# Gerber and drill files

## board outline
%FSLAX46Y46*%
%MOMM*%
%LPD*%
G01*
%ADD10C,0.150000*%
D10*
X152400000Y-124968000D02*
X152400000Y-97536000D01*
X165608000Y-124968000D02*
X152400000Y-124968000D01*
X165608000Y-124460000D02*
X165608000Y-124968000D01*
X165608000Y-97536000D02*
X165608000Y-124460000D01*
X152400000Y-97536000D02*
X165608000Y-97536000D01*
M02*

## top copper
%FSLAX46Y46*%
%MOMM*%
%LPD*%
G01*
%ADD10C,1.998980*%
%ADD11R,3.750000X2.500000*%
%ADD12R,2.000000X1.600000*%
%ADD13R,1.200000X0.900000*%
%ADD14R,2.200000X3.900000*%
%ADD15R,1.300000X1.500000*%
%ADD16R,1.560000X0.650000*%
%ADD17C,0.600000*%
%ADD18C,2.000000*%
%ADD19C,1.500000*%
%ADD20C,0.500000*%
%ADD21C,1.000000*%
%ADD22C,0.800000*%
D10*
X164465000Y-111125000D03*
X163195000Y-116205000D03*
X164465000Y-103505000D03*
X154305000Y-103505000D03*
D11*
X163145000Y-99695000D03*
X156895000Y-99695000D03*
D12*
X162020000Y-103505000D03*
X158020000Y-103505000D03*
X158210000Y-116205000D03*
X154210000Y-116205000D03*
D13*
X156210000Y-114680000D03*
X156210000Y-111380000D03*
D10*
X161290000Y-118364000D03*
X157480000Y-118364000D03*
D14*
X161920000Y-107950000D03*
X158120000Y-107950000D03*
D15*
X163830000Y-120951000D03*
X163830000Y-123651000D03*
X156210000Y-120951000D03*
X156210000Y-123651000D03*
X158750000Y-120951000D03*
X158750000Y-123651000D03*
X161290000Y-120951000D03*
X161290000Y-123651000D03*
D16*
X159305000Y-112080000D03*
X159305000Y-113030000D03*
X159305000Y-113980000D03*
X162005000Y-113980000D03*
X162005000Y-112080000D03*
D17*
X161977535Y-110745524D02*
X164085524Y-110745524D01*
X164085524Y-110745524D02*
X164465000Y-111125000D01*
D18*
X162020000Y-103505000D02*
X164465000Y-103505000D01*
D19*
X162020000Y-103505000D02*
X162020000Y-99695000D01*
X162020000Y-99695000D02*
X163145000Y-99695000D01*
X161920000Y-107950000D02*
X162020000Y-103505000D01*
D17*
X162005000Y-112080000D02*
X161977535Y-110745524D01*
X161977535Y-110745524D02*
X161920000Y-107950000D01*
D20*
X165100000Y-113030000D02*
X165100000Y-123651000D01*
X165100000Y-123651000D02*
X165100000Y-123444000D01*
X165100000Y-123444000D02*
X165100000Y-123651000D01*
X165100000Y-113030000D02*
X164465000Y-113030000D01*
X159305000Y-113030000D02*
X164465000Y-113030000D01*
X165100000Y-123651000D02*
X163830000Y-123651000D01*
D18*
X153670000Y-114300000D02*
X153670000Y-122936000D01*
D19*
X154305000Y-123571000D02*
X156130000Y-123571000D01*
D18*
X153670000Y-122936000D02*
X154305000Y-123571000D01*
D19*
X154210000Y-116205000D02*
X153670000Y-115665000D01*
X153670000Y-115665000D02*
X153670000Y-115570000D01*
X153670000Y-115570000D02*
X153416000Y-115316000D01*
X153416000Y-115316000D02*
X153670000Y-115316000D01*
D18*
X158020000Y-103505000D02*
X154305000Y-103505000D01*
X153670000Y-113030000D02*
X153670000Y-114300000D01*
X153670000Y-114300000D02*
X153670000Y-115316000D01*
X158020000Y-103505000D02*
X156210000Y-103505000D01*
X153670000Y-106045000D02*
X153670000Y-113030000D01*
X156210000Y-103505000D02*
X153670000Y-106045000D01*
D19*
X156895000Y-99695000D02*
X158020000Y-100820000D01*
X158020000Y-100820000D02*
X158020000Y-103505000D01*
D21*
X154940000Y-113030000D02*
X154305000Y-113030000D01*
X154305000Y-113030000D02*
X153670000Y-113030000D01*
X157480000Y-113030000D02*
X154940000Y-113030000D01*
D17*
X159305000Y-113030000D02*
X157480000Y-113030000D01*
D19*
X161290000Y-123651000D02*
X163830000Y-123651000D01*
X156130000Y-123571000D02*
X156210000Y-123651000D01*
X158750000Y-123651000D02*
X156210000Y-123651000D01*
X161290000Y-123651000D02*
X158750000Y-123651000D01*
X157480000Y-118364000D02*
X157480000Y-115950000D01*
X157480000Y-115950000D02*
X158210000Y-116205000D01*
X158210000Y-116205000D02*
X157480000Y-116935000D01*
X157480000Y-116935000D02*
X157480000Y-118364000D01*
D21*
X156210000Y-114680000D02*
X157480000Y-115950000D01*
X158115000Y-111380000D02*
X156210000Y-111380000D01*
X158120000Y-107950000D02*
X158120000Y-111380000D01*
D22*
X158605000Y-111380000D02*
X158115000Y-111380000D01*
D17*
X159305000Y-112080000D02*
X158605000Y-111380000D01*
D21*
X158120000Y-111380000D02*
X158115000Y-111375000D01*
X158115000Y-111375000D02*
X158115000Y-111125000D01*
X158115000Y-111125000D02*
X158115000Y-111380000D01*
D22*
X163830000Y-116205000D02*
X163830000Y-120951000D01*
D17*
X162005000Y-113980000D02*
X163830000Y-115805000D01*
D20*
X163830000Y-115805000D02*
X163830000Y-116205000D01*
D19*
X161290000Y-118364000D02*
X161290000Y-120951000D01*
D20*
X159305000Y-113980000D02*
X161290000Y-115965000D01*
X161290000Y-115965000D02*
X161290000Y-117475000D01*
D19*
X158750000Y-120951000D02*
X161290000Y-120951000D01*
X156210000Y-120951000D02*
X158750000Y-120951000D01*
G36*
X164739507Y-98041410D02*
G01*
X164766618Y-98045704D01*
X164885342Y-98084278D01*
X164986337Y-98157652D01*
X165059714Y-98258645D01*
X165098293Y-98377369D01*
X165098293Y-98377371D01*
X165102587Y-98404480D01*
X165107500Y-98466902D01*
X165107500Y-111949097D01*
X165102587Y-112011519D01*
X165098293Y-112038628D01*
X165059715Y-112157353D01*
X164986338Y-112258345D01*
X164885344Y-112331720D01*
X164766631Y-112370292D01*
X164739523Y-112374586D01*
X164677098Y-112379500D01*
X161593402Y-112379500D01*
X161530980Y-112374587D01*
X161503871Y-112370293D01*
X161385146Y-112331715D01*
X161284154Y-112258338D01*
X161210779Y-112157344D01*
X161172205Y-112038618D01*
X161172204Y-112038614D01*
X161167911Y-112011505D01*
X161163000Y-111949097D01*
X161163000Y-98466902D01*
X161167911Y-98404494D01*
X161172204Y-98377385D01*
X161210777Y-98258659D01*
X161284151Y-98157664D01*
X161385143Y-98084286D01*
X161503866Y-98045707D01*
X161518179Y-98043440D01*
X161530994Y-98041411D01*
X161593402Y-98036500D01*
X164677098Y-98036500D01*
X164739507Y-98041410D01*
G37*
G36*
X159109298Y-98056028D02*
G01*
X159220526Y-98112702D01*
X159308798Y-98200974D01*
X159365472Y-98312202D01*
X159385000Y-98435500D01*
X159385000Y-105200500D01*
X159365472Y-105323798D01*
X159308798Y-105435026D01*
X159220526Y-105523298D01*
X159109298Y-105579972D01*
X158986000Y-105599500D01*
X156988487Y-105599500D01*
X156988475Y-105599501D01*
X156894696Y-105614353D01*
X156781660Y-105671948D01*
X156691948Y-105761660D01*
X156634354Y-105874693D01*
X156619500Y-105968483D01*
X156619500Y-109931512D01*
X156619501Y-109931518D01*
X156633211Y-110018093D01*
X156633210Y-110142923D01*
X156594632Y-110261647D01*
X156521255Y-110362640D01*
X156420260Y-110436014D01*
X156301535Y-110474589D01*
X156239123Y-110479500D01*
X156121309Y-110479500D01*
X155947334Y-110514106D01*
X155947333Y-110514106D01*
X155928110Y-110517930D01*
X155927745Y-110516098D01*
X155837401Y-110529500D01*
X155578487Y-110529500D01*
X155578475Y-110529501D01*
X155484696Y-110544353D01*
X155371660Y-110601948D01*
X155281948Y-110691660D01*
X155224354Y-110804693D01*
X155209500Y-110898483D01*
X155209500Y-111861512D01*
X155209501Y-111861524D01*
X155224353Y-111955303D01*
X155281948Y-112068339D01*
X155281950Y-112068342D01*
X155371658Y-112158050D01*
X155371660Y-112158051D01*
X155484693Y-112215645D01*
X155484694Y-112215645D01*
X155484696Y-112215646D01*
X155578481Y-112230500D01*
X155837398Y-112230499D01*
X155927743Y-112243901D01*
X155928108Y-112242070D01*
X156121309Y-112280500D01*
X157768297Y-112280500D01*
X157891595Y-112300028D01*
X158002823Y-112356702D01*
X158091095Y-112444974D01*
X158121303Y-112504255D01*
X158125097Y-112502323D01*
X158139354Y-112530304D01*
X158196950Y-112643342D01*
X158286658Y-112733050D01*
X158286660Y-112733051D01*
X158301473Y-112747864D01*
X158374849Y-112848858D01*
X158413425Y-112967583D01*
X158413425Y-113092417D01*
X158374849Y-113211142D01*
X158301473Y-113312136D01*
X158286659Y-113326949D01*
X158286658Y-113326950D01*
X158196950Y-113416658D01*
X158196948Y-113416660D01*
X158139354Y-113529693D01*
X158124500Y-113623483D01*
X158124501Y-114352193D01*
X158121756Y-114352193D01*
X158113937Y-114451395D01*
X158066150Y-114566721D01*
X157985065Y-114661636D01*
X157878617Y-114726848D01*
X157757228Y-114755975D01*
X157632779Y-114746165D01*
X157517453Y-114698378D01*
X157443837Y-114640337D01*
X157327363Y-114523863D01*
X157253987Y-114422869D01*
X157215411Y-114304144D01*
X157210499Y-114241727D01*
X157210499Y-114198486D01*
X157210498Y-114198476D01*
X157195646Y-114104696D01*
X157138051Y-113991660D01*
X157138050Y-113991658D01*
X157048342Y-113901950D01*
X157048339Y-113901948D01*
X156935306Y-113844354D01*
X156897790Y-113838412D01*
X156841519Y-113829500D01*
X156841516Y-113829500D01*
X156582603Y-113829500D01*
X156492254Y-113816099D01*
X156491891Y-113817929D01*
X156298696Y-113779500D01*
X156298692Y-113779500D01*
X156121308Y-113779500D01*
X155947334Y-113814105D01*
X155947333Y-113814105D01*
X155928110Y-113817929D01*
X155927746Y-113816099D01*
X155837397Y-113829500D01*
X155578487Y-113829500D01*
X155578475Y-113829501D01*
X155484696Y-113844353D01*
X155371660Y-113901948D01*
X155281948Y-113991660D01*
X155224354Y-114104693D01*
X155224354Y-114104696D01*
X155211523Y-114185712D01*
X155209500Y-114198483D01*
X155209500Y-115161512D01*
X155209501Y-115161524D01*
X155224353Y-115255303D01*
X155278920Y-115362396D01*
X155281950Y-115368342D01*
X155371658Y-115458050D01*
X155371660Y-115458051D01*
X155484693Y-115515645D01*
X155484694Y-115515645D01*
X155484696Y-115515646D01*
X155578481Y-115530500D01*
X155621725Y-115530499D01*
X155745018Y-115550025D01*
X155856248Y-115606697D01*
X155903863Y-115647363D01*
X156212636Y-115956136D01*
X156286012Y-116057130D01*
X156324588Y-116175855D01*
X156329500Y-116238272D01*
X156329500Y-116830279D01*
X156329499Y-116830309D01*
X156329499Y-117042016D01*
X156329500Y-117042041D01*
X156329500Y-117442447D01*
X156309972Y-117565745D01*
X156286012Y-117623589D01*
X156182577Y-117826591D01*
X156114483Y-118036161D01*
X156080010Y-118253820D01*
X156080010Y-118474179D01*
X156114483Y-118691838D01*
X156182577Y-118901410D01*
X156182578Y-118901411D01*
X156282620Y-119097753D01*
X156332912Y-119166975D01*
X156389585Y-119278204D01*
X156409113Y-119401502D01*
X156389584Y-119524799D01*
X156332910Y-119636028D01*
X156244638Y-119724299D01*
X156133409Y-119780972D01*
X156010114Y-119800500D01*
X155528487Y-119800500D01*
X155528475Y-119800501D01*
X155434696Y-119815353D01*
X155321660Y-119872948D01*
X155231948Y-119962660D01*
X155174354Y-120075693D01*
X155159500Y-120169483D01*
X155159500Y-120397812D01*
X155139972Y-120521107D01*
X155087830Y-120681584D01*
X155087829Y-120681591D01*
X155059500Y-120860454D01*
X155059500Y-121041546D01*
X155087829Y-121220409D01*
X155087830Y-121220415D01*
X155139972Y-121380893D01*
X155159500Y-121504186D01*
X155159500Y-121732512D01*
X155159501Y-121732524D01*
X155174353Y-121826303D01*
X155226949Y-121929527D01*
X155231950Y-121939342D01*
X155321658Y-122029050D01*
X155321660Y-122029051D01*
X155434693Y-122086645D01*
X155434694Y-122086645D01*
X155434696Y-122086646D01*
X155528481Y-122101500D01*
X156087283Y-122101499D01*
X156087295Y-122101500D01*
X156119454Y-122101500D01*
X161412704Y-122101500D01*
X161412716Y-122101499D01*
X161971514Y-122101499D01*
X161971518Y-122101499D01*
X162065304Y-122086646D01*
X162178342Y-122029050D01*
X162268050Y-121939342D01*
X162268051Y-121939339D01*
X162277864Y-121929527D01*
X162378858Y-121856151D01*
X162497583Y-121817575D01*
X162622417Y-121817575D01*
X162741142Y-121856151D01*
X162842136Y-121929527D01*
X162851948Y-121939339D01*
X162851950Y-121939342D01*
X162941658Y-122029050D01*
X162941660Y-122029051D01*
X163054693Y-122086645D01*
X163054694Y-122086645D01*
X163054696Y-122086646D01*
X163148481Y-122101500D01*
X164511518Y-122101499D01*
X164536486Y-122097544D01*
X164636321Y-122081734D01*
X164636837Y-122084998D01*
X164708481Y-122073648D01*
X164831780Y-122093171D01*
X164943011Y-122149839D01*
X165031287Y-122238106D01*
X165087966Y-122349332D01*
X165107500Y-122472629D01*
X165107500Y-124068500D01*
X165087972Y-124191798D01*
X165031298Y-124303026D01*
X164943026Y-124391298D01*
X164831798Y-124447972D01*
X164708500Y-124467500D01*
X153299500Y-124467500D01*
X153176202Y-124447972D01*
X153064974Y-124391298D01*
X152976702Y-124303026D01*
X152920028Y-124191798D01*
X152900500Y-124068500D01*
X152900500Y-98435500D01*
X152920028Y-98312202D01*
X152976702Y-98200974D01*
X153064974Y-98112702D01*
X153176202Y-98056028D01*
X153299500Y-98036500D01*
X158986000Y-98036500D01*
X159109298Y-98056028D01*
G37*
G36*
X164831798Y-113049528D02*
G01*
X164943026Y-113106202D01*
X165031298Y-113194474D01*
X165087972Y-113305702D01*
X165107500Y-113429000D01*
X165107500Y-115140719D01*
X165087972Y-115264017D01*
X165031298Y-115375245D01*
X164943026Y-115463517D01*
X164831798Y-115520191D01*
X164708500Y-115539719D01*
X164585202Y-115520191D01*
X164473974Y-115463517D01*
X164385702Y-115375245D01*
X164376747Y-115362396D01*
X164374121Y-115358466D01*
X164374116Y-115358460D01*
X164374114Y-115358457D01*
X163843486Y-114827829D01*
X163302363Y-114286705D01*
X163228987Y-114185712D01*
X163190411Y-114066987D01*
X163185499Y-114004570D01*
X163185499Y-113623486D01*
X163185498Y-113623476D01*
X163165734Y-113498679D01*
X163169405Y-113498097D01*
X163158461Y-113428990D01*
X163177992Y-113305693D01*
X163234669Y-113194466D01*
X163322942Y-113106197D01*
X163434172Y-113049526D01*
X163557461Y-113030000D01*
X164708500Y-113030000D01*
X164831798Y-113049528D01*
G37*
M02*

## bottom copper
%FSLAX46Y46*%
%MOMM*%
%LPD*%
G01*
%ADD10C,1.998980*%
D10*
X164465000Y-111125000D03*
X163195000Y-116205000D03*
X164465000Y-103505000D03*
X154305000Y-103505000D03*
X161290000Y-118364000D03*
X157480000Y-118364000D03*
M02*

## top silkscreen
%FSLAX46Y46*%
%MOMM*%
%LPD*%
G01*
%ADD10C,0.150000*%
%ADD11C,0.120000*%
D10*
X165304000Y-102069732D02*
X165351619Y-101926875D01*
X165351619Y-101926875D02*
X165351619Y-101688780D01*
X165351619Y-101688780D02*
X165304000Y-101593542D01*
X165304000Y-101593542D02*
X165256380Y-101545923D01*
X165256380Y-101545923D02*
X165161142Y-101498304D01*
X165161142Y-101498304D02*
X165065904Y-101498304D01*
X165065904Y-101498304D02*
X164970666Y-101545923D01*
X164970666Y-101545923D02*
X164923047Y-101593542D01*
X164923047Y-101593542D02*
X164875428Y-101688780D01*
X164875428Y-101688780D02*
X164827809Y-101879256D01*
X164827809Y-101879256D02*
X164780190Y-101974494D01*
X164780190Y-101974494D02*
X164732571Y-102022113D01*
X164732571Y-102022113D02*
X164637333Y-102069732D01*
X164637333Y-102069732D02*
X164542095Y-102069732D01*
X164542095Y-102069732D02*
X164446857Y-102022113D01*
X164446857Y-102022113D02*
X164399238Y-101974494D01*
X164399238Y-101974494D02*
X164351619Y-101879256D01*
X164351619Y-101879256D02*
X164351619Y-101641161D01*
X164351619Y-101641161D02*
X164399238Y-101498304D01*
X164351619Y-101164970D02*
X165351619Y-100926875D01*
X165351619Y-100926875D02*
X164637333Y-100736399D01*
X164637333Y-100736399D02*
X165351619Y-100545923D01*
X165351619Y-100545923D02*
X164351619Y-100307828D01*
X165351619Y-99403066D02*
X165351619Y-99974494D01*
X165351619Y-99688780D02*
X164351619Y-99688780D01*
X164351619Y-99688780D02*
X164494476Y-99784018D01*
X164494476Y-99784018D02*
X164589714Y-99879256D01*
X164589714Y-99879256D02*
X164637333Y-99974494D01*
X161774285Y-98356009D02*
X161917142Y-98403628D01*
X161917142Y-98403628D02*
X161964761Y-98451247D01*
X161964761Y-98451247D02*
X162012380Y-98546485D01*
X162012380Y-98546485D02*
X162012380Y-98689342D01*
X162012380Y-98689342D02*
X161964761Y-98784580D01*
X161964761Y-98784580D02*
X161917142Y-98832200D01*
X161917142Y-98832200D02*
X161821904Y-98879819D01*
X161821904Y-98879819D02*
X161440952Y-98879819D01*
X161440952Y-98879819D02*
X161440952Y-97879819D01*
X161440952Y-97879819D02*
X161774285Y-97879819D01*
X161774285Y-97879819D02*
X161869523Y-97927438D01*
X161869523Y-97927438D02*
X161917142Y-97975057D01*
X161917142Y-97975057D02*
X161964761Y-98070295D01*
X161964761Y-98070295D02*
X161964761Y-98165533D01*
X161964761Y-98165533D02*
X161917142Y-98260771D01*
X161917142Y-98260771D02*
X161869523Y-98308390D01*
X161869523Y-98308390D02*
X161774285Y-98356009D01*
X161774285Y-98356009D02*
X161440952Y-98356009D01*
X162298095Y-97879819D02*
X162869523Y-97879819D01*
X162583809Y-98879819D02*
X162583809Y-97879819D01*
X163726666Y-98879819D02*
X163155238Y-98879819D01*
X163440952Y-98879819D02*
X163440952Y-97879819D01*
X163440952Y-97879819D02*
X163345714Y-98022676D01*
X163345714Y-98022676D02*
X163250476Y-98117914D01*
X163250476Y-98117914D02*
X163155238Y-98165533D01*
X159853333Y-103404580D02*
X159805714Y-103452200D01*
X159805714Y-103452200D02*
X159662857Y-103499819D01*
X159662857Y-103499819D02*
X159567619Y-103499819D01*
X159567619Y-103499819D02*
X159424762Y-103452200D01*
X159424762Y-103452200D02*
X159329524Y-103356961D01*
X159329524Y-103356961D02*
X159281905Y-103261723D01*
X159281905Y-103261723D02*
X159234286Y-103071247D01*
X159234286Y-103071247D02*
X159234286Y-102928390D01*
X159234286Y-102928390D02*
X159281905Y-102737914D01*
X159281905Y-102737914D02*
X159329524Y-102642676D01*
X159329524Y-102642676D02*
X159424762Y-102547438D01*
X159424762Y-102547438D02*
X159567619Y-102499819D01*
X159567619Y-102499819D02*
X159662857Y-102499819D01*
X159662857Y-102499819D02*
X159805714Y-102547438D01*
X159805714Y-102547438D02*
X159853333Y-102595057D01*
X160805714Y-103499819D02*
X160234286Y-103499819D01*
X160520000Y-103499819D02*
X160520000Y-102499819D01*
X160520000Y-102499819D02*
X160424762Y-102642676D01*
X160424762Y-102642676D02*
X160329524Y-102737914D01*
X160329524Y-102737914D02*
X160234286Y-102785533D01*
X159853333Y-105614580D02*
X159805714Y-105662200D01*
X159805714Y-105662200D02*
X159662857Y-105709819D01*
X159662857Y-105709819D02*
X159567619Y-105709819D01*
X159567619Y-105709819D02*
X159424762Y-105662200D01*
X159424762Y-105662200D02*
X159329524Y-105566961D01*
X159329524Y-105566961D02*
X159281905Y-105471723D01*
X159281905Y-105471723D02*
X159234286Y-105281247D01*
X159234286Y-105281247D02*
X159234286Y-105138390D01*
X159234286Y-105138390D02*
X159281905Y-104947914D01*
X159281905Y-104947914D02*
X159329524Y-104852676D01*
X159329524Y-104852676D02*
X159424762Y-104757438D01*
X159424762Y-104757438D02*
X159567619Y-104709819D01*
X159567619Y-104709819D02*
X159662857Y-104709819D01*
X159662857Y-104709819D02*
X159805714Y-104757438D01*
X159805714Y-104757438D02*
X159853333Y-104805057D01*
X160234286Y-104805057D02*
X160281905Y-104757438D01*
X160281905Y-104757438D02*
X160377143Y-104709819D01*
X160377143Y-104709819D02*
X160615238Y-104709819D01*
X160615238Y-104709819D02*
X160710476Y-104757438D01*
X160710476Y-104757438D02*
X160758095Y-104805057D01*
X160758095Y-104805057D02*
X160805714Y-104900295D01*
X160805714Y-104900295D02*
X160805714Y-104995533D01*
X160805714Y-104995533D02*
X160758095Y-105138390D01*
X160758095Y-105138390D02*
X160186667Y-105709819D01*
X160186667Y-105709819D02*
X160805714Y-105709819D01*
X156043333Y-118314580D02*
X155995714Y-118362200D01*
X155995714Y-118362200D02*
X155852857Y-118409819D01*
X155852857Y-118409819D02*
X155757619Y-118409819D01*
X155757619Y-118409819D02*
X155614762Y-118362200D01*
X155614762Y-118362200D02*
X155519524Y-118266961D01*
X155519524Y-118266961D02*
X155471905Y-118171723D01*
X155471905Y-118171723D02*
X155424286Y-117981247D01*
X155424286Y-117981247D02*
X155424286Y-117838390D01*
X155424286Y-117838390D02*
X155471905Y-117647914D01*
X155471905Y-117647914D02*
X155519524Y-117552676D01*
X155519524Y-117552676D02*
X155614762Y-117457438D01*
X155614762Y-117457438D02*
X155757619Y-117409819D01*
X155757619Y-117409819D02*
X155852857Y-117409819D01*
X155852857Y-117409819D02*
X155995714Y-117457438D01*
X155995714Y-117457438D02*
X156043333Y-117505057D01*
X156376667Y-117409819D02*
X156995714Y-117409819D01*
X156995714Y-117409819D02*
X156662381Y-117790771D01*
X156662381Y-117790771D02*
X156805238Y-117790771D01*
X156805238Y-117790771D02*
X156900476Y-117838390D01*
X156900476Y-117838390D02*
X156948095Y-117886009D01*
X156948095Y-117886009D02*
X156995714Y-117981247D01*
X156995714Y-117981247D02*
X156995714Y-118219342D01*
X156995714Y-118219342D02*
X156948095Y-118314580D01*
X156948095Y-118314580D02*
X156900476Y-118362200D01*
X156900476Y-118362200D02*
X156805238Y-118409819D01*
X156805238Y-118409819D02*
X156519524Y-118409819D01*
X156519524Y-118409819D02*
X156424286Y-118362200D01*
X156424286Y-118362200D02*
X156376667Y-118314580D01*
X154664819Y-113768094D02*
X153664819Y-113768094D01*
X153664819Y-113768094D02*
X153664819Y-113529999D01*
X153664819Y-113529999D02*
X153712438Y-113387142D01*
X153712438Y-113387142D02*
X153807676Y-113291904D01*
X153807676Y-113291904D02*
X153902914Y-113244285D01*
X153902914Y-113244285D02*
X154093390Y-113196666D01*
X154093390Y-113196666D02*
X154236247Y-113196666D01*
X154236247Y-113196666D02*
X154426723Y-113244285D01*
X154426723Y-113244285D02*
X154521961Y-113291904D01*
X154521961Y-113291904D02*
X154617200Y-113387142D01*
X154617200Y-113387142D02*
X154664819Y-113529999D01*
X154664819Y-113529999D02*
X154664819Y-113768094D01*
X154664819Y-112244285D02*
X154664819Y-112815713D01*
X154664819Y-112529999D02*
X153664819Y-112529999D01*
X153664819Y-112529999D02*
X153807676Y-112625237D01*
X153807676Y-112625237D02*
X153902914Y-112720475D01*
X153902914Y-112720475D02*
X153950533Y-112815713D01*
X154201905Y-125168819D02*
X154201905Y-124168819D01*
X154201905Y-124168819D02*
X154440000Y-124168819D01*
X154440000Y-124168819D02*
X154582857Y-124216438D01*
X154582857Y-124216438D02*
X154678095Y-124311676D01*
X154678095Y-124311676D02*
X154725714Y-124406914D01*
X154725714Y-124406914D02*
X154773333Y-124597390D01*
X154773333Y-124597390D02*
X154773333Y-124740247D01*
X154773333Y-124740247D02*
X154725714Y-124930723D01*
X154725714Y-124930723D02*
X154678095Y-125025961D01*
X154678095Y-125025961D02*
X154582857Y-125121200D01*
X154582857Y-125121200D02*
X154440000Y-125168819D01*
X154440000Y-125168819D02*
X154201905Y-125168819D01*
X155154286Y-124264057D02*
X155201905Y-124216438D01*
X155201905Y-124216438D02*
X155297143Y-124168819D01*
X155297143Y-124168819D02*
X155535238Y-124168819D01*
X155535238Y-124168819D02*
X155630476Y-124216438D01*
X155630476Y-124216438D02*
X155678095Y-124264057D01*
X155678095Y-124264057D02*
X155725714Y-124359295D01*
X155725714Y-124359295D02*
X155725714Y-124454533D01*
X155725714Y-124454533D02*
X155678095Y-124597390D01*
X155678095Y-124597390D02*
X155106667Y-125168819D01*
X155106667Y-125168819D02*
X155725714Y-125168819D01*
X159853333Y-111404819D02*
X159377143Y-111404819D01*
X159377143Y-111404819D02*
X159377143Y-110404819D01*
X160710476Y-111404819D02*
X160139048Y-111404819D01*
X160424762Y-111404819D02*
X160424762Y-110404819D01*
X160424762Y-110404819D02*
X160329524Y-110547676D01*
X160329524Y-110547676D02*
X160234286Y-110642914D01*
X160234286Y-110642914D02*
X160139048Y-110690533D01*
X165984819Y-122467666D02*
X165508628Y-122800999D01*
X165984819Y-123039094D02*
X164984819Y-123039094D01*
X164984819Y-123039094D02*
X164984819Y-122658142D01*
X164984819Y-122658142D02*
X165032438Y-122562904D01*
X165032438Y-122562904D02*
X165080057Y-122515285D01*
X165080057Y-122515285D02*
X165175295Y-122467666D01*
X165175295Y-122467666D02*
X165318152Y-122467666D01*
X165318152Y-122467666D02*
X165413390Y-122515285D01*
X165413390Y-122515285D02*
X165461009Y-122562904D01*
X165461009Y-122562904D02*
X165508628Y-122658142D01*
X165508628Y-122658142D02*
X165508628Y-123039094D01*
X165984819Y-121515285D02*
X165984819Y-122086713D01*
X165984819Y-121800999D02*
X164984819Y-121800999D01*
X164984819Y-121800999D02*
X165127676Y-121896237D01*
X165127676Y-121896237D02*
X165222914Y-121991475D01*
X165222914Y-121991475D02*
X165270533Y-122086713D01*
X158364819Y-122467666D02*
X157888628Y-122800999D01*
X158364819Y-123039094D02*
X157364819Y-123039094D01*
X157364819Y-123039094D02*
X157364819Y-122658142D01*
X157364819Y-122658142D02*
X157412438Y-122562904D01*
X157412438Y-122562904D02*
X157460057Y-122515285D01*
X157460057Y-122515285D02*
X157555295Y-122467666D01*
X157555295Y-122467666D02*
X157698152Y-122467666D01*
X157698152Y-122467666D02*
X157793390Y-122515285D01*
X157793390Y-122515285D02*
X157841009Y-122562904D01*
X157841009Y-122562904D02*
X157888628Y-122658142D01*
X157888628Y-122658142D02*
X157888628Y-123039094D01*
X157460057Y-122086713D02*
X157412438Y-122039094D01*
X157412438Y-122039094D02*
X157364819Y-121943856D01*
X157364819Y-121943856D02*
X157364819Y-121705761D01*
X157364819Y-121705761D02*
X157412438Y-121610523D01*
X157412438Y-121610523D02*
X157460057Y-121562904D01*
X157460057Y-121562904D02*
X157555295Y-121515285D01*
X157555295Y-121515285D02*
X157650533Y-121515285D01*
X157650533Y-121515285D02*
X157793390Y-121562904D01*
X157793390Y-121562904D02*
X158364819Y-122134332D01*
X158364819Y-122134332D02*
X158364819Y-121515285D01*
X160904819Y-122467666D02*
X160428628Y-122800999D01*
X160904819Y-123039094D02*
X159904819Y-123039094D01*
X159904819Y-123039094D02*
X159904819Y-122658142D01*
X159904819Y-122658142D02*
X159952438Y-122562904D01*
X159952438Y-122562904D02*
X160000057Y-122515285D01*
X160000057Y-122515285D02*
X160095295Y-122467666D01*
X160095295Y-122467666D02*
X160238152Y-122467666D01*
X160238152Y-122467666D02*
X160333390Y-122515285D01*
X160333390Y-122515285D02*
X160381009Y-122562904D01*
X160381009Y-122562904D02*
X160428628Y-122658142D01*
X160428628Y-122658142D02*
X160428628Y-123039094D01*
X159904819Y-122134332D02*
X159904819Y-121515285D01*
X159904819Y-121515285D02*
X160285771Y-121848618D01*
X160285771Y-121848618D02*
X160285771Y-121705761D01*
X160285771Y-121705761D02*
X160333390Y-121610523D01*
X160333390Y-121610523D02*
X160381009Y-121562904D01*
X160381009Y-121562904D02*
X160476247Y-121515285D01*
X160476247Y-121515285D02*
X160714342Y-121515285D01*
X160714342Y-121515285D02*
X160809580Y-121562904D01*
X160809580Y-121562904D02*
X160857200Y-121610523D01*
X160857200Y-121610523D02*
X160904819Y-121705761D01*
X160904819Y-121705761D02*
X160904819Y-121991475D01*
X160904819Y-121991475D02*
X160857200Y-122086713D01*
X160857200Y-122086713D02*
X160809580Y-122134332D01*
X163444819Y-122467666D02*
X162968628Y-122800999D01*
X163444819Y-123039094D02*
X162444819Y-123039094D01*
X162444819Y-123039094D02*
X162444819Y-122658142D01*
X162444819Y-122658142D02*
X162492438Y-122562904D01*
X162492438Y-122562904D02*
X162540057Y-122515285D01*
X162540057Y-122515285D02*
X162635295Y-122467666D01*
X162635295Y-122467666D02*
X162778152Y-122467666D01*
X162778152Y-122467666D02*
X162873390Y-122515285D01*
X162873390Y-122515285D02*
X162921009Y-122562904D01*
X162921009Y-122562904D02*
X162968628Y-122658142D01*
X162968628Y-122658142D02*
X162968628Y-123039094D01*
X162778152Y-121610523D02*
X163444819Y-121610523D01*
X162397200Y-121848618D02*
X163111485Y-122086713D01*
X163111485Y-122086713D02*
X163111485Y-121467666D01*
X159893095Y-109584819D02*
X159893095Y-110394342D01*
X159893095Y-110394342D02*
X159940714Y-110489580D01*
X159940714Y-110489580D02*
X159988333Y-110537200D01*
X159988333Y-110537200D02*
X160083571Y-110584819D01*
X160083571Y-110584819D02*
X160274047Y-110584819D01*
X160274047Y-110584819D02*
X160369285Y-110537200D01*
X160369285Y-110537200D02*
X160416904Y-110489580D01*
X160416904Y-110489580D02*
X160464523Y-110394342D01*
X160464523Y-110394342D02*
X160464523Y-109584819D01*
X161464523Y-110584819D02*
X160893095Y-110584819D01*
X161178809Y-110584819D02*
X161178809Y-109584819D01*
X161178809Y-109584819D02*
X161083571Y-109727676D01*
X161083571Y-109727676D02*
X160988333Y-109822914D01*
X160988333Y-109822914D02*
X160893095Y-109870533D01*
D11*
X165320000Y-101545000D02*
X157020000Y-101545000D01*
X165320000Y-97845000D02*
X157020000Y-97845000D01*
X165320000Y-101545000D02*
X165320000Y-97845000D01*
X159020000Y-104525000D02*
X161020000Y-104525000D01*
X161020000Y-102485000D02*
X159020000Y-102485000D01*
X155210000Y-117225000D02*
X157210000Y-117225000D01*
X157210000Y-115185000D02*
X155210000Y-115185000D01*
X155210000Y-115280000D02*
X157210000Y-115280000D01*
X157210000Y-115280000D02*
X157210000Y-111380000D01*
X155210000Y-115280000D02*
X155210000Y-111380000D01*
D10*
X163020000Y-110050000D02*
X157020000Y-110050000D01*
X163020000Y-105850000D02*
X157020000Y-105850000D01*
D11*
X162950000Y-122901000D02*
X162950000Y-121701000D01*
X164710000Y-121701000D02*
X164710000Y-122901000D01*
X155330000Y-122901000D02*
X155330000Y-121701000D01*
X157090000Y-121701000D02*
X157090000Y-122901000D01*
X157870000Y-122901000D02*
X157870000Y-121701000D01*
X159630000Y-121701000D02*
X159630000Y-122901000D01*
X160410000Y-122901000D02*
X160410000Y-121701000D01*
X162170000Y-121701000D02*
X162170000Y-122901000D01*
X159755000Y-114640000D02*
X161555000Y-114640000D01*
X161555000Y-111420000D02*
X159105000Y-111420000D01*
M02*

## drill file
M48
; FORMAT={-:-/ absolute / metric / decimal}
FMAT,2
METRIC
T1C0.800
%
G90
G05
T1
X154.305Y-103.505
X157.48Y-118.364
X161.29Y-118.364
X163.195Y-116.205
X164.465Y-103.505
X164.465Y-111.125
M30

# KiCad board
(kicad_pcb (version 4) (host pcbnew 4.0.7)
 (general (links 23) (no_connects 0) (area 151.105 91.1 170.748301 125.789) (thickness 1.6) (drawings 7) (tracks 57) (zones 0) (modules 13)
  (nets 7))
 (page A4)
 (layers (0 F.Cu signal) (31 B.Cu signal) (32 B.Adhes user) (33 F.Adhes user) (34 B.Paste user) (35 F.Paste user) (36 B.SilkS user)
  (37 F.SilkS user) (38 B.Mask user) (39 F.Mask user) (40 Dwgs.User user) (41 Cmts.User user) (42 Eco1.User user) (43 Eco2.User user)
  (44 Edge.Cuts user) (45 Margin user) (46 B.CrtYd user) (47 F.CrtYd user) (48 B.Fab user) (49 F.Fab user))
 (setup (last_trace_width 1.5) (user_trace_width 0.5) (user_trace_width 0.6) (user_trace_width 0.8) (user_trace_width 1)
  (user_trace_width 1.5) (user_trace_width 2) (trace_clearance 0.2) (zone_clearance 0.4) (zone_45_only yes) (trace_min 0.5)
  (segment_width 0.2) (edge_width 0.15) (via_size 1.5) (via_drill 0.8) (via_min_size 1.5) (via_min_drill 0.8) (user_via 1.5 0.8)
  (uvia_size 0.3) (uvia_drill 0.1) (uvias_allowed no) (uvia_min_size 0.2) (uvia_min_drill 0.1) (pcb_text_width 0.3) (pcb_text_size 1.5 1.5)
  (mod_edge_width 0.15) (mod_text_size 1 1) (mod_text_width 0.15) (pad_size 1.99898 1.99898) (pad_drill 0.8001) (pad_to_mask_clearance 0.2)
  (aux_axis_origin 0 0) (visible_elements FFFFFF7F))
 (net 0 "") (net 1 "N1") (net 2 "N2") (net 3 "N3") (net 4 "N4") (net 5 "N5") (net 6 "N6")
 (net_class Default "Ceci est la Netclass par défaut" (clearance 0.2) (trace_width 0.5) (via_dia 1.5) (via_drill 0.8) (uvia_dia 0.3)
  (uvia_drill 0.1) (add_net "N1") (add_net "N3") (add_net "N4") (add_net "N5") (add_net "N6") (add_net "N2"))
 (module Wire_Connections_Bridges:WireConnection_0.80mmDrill (layer F.Cu) (at 165.1 95.885 270)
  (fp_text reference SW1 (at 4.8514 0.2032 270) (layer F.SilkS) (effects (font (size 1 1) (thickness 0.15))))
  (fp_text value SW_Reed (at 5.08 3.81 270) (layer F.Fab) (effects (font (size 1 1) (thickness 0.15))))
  (pad 1 thru_hole circle (at 15.24 0.635 270) (size 1.99898 1.99898) (drill 0.8001) (layers *.Cu *.Mask) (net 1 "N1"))
  (pad 2 thru_hole circle (at 20.32 1.905 270) (size 1.99898 1.99898) (drill 0.8001) (layers *.Cu *.Mask) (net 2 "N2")))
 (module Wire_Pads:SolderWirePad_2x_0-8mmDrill (layer F.Cu) (at 162.56 94.615 180)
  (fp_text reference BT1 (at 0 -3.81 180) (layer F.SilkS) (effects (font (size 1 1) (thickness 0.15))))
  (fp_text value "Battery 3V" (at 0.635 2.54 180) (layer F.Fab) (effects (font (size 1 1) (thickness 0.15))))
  (pad 1 thru_hole circle (at -1.905 -8.89 180) (size 1.99898 1.99898) (drill 0.8001) (layers *.Cu *.Mask) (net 1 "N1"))
  (pad 2 thru_hole circle (at 8.255 -8.89 180) (size 1.99898 1.99898) (drill 0.8001) (layers *.Cu *.Mask) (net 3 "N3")))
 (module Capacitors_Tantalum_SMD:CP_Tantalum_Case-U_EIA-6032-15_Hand (layer F.Cu) (at 160.02 99.695 180)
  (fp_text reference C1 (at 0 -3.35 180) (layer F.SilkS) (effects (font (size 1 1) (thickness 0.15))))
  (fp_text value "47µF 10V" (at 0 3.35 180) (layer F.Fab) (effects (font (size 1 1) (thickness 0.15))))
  (fp_line (start -5.3 -1.85) (end 3 -1.85) (layer F.SilkS) (width 0.12))
  (fp_line (start -5.3 1.85) (end 3 1.85) (layer F.SilkS) (width 0.12))
  (fp_line (start -5.3 -1.85) (end -5.3 1.85) (layer F.SilkS) (width 0.12))
  (pad 1 smd rect (at -3.125 0 180) (size 3.75 2.5) (layers F.Cu F.Paste F.Mask) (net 1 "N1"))
  (pad 2 smd rect (at 3.125 0 180) (size 3.75 2.5) (layers F.Cu F.Paste F.Mask) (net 3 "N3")))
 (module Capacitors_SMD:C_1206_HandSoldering (layer F.Cu) (at 160.02 103.505 180)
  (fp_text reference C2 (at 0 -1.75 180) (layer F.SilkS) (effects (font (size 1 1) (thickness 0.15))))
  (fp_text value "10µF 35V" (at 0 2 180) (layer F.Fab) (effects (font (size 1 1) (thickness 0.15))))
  (fp_line (start 1 -1.02) (end -1 -1.02) (layer F.SilkS) (width 0.12))
  (fp_line (start -1 1.02) (end 1 1.02) (layer F.SilkS) (width 0.12))
  (pad 1 smd rect (at -2 0 180) (size 2 1.6) (layers F.Cu F.Paste F.Mask) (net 1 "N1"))
  (pad 2 smd rect (at 2 0 180) (size 2 1.6) (layers F.Cu F.Paste F.Mask) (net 3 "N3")))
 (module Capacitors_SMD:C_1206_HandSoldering (layer F.Cu) (at 156.21 116.205 180)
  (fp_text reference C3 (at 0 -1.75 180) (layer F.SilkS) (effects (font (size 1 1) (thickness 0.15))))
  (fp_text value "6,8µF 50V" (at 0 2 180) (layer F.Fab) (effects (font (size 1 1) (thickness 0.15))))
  (fp_line (start 1 -1.02) (end -1 -1.02) (layer F.SilkS) (width 0.12))
  (fp_line (start -1 1.02) (end 1 1.02) (layer F.SilkS) (width 0.12))
  (pad 1 smd rect (at -2 0 180) (size 2 1.6) (layers F.Cu F.Paste F.Mask) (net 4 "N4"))
  (pad 2 smd rect (at 2 0 180) (size 2 1.6) (layers F.Cu F.Paste F.Mask) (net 3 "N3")))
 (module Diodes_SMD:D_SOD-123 (layer F.Cu) (at 156.21 113.03 90)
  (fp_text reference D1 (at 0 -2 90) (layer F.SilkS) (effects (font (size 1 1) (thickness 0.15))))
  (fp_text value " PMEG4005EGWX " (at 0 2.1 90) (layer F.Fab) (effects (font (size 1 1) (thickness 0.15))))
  (fp_line (start -2.25 -1) (end -2.25 1) (layer F.SilkS) (width 0.12))
  (fp_line (start -2.25 1) (end 1.65 1) (layer F.SilkS) (width 0.12))
  (fp_line (start -2.25 -1) (end 1.65 -1) (layer F.SilkS) (width 0.12))
  (pad 1 smd rect (at -1.65 0 90) (size 0.9 1.2) (layers F.Cu F.Paste F.Mask) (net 4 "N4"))
  (pad 2 smd rect (at 1.65 0 90) (size 0.9 1.2) (layers F.Cu F.Paste F.Mask) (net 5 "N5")))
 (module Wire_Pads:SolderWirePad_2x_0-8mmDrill (layer F.Cu) (at 154.94 120.904 180)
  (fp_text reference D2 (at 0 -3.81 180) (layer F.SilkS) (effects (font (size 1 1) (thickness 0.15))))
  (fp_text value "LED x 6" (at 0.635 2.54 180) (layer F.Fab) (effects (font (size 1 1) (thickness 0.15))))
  (pad 1 thru_hole circle (at -6.35 2.54 180) (size 1.99898 1.99898) (drill 0.8001) (layers *.Cu *.Mask) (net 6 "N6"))
  (pad 2 thru_hole circle (at -2.54 2.54 180) (size 1.99898 1.99898) (drill 0.8001) (layers *.Cu *.Mask) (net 4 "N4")))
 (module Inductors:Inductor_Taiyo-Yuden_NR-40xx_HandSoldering (layer F.Cu) (at 160.02 107.95 180)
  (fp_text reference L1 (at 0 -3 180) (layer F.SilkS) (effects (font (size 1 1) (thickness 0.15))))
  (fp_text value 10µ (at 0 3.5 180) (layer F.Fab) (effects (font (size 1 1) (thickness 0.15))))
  (fp_line (start -3 -2.1) (end 3 -2.1) (layer F.SilkS) (width 0.15))
  (fp_line (start -3 2.1) (end 3 2.1) (layer F.SilkS) (width 0.15))
  (pad 1 smd rect (at -1.9 0 180) (size 2.2 3.9) (layers F.Cu F.Paste F.Mask) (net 1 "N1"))
  (pad 2 smd rect (at 1.9 0 180) (size 2.2 3.9) (layers F.Cu F.Paste F.Mask) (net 5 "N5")))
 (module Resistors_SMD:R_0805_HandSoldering (layer F.Cu) (at 163.83 122.301 270)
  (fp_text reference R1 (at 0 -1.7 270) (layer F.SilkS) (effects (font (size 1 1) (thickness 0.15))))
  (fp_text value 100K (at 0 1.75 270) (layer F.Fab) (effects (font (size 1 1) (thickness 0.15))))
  (fp_line (start 0.6 0.88) (end -0.6 0.88) (layer F.SilkS) (width 0.12))
  (fp_line (start -0.6 -0.88) (end 0.6 -0.88) (layer F.SilkS) (width 0.12))
  (pad 1 smd rect (at -1.35 0 270) (size 1.5 1.3) (layers F.Cu F.Paste F.Mask) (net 2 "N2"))
  (pad 2 smd rect (at 1.35 0 270) (size 1.5 1.3) (layers F.Cu F.Paste F.Mask) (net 3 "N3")))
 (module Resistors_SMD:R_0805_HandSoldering (layer F.Cu) (at 156.21 122.301 270)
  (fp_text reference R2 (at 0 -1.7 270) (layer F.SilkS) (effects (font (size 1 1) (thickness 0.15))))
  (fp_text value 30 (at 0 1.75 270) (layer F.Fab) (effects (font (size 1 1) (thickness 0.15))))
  (fp_line (start 0.6 0.88) (end -0.6 0.88) (layer F.SilkS) (width 0.12))
  (fp_line (start -0.6 -0.88) (end 0.6 -0.88) (layer F.SilkS) (width 0.12))
  (pad 1 smd rect (at -1.35 0 270) (size 1.5 1.3) (layers F.Cu F.Paste F.Mask) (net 6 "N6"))
  (pad 2 smd rect (at 1.35 0 270) (size 1.5 1.3) (layers F.Cu F.Paste F.Mask) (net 3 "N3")))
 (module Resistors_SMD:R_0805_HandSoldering (layer F.Cu) (at 158.75 122.301 270)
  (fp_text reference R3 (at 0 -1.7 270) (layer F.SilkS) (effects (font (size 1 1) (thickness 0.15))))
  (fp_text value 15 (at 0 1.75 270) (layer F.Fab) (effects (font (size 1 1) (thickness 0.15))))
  (fp_line (start 0.6 0.88) (end -0.6 0.88) (layer F.SilkS) (width 0.12))
  (fp_line (start -0.6 -0.88) (end 0.6 -0.88) (layer F.SilkS) (width 0.12))
  (pad 1 smd rect (at -1.35 0 270) (size 1.5 1.3) (layers F.Cu F.Paste F.Mask) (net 6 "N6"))
  (pad 2 smd rect (at 1.35 0 270) (size 1.5 1.3) (layers F.Cu F.Paste F.Mask) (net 3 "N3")))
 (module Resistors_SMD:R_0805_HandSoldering (layer F.Cu) (at 161.29 122.301 270)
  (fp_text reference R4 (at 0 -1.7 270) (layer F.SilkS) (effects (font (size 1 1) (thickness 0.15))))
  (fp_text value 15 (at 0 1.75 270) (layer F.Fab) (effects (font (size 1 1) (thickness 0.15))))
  (fp_line (start 0.6 0.88) (end -0.6 0.88) (layer F.SilkS) (width 0.12))
  (fp_line (start -0.6 -0.88) (end 0.6 -0.88) (layer F.SilkS) (width 0.12))
  (pad 1 smd rect (at -1.35 0 270) (size 1.5 1.3) (layers F.Cu F.Paste F.Mask) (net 6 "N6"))
  (pad 2 smd rect (at 1.35 0 270) (size 1.5 1.3) (layers F.Cu F.Paste F.Mask) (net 3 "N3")))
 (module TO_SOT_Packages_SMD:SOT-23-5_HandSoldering (layer F.Cu) (at 160.655 113.03)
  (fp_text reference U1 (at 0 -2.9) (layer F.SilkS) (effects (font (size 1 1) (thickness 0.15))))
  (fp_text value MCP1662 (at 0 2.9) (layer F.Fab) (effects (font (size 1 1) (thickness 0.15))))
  (fp_line (start -0.9 1.61) (end 0.9 1.61) (layer F.SilkS) (width 0.12))
  (fp_line (start 0.9 -1.61) (end -1.55 -1.61) (layer F.SilkS) (width 0.12))
  (pad 1 smd rect (at -1.35 -0.95) (size 1.56 0.65) (layers F.Cu F.Paste F.Mask) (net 5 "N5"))
  (pad 2 smd rect (at -1.35 0) (size 1.56 0.65) (layers F.Cu F.Paste F.Mask) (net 3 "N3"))
  (pad 3 smd rect (at -1.35 0.95) (size 1.56 0.65) (layers F.Cu F.Paste F.Mask) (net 6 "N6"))
  (pad 4 smd rect (at 1.35 0.95) (size 1.56 0.65) (layers F.Cu F.Paste F.Mask) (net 2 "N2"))
  (pad 5 smd rect (at 1.35 -0.95) (size 1.56 0.65) (layers F.Cu F.Paste F.Mask) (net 1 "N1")))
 (gr_line (start 152.4 124.968) (end 152.4 97.536) (angle 90) (layer Edge.Cuts) (width 0.15))
 (gr_line (start 165.608 124.968) (end 152.4 124.968) (angle 90) (layer Edge.Cuts) (width 0.15))
 (gr_line (start 165.608 124.46) (end 165.608 124.968) (angle 90) (layer Edge.Cuts) (width 0.15))
 (gr_line (start 165.608 97.536) (end 165.608 124.46) (angle 90) (layer Edge.Cuts) (width 0.15))
 (gr_line (start 152.4 97.536) (end 165.608 97.536) (angle 90) (layer Edge.Cuts) (width 0.15))
 (segment (start 161.977535 110.745524) (end 164.085524 110.745524) (width 0.6) (layer F.Cu) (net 1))
 (segment (start 164.085524 110.745524) (end 164.465 111.125) (width 0.6) (layer F.Cu) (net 1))
 (segment (start 162.02 103.505) (end 164.465 103.505) (width 2) (layer F.Cu) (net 1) (status 20))
 (segment (start 162.02 103.505) (end 162.02 99.695) (width 1.5) (layer F.Cu) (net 1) (status 10))
 (segment (start 162.02 99.695) (end 163.145 99.695) (width 1.5) (layer F.Cu) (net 1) (status 30))
 (segment (start 161.92 107.95) (end 162.02 103.505) (width 1.5) (layer F.Cu) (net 1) (status 10))
 (segment (start 162.005 112.08) (end 161.977535 110.745524) (width 0.6) (layer F.Cu) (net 1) (status 20))
 (segment (start 161.977535 110.745524) (end 161.92 107.95) (width 0.6) (layer F.Cu) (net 1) (status 20))
 (segment (start 165.1 113.03) (end 165.1 123.651) (width 0.5) (layer F.Cu) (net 3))
 (segment (start 165.1 123.651) (end 165.1 123.444) (width 0.5) (layer F.Cu) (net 3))
 (segment (start 165.1 123.444) (end 165.1 123.651) (width 0.5) (layer F.Cu) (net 3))
 (segment (start 165.1 113.03) (end 164.465 113.03) (width 0.5) (layer F.Cu) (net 3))
 (segment (start 159.305 113.03) (end 164.465 113.03) (width 0.5) (layer F.Cu) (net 3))
 (segment (start 165.1 123.651) (end 163.83 123.651) (width 0.5) (layer F.Cu) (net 3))
 (segment (start 153.67 114.3) (end 153.67 122.936) (width 2) (layer F.Cu) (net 3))
 (segment (start 154.305 123.571) (end 156.13 123.571) (width 1.5) (layer F.Cu) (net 3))
 (segment (start 153.67 122.936) (end 154.305 123.571) (width 2) (layer F.Cu) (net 3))
 (segment (start 154.21 116.205) (end 153.67 115.665) (width 1.5) (layer F.Cu) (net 3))
 (segment (start 153.67 115.665) (end 153.67 115.57) (width 1.5) (layer F.Cu) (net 3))
 (segment (start 153.67 115.57) (end 153.416 115.316) (width 1.5) (layer F.Cu) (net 3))
 (segment (start 153.416 115.316) (end 153.67 115.316) (width 1.5) (layer F.Cu) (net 3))
 (segment (start 158.02 103.505) (end 154.305 103.505) (width 2) (layer F.Cu) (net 3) (status 20))
 (segment (start 153.67 113.03) (end 153.67 114.3) (width 2) (layer F.Cu) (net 3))
 (segment (start 153.67 114.3) (end 153.67 115.316) (width 2) (layer F.Cu) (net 3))
 (segment (start 158.02 103.505) (end 156.21 103.505) (width 2) (layer F.Cu) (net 3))
 (segment (start 153.67 106.045) (end 153.67 113.03) (width 2) (layer F.Cu) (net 3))
 (segment (start 156.21 103.505) (end 153.67 106.045) (width 2) (layer F.Cu) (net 3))
 (segment (start 156.895 99.695) (end 158.02 100.82) (width 1.5) (layer F.Cu) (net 3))
 (segment (start 158.02 100.82) (end 158.02 103.505) (width 1.5) (layer F.Cu) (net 3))
 (segment (start 154.94 113.03) (end 154.305 113.03) (width 1) (layer F.Cu) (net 3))
 (segment (start 154.305 113.03) (end 153.67 113.03) (width 1) (layer F.Cu) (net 3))
 (segment (start 157.48 113.03) (end 154.94 113.03) (width 1) (layer F.Cu) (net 3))
 (segment (start 159.305 113.03) (end 157.48 113.03) (width 0.6) (layer F.Cu) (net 3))
 (segment (start 161.29 123.651) (end 163.83 123.651) (width 1.5) (layer F.Cu) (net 3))
 (segment (start 156.13 123.571) (end 156.21 123.651) (width 1.5) (layer F.Cu) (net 3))
 (segment (start 158.75 123.651) (end 156.21 123.651) (width 1.5) (layer F.Cu) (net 3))
 (segment (start 161.29 123.651) (end 158.75 123.651) (width 1.5) (layer F.Cu) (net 3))
 (segment (start 157.48 118.364) (end 157.48 115.95) (width 1.5) (layer F.Cu) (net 4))
 (segment (start 157.48 115.95) (end 158.21 116.205) (width 1.5) (layer F.Cu) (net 4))
 (segment (start 158.21 116.205) (end 157.48 116.935) (width 1.5) (layer F.Cu) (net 4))
 (segment (start 157.48 116.935) (end 157.48 118.364) (width 1.5) (layer F.Cu) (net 4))
 (segment (start 156.21 114.68) (end 157.48 115.95) (width 1) (layer F.Cu) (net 4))
 (segment (start 158.115 111.38) (end 156.21 111.38) (width 1) (layer F.Cu) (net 5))
 (segment (start 158.12 107.95) (end 158.12 111.38) (width 1) (layer F.Cu) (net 5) (status 10))
 (segment (start 158.605 111.38) (end 158.115 111.38) (width 0.8) (layer F.Cu) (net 5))
 (segment (start 159.305 112.08) (end 158.605 111.38) (width 0.6) (layer F.Cu) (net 5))
 (segment (start 158.12 111.38) (end 158.115 111.375) (width 1) (layer F.Cu) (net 5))
 (segment (start 158.115 111.375) (end 158.115 111.125) (width 1) (layer F.Cu) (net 5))
 (segment (start 158.115 111.125) (end 158.115 111.38) (width 1) (layer F.Cu) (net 5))
 (segment (start 163.83 116.205) (end 163.83 120.951) (width 0.8) (layer F.Cu) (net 2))
 (segment (start 162.005 113.98) (end 163.83 115.805) (width 0.6) (layer F.Cu) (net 2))
 (segment (start 163.83 115.805) (end 163.83 116.205) (width 0.5) (layer F.Cu) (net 2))
 (segment (start 161.29 118.364) (end 161.29 120.951) (width 1.5) (layer F.Cu) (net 6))
 (segment (start 159.305 113.98) (end 161.29 115.965) (width 0.5) (layer F.Cu) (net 6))
 (segment (start 161.29 115.965) (end 161.29 117.475) (width 0.5) (layer F.Cu) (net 6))
 (segment (start 158.75 120.951) (end 161.29 120.951) (width 1.5) (layer F.Cu) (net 6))
 (segment (start 156.21 120.951) (end 158.75 120.951) (width 1.5) (layer F.Cu) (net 6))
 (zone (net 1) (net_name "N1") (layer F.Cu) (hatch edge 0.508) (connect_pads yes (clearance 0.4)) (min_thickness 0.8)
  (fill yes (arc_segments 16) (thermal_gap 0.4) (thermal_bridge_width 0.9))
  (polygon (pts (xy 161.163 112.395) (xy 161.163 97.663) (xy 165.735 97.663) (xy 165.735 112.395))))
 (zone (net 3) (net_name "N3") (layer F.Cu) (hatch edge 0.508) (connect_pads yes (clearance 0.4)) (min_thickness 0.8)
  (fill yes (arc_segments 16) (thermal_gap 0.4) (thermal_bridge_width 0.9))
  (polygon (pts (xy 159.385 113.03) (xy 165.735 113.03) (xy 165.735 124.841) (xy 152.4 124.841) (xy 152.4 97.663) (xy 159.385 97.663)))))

